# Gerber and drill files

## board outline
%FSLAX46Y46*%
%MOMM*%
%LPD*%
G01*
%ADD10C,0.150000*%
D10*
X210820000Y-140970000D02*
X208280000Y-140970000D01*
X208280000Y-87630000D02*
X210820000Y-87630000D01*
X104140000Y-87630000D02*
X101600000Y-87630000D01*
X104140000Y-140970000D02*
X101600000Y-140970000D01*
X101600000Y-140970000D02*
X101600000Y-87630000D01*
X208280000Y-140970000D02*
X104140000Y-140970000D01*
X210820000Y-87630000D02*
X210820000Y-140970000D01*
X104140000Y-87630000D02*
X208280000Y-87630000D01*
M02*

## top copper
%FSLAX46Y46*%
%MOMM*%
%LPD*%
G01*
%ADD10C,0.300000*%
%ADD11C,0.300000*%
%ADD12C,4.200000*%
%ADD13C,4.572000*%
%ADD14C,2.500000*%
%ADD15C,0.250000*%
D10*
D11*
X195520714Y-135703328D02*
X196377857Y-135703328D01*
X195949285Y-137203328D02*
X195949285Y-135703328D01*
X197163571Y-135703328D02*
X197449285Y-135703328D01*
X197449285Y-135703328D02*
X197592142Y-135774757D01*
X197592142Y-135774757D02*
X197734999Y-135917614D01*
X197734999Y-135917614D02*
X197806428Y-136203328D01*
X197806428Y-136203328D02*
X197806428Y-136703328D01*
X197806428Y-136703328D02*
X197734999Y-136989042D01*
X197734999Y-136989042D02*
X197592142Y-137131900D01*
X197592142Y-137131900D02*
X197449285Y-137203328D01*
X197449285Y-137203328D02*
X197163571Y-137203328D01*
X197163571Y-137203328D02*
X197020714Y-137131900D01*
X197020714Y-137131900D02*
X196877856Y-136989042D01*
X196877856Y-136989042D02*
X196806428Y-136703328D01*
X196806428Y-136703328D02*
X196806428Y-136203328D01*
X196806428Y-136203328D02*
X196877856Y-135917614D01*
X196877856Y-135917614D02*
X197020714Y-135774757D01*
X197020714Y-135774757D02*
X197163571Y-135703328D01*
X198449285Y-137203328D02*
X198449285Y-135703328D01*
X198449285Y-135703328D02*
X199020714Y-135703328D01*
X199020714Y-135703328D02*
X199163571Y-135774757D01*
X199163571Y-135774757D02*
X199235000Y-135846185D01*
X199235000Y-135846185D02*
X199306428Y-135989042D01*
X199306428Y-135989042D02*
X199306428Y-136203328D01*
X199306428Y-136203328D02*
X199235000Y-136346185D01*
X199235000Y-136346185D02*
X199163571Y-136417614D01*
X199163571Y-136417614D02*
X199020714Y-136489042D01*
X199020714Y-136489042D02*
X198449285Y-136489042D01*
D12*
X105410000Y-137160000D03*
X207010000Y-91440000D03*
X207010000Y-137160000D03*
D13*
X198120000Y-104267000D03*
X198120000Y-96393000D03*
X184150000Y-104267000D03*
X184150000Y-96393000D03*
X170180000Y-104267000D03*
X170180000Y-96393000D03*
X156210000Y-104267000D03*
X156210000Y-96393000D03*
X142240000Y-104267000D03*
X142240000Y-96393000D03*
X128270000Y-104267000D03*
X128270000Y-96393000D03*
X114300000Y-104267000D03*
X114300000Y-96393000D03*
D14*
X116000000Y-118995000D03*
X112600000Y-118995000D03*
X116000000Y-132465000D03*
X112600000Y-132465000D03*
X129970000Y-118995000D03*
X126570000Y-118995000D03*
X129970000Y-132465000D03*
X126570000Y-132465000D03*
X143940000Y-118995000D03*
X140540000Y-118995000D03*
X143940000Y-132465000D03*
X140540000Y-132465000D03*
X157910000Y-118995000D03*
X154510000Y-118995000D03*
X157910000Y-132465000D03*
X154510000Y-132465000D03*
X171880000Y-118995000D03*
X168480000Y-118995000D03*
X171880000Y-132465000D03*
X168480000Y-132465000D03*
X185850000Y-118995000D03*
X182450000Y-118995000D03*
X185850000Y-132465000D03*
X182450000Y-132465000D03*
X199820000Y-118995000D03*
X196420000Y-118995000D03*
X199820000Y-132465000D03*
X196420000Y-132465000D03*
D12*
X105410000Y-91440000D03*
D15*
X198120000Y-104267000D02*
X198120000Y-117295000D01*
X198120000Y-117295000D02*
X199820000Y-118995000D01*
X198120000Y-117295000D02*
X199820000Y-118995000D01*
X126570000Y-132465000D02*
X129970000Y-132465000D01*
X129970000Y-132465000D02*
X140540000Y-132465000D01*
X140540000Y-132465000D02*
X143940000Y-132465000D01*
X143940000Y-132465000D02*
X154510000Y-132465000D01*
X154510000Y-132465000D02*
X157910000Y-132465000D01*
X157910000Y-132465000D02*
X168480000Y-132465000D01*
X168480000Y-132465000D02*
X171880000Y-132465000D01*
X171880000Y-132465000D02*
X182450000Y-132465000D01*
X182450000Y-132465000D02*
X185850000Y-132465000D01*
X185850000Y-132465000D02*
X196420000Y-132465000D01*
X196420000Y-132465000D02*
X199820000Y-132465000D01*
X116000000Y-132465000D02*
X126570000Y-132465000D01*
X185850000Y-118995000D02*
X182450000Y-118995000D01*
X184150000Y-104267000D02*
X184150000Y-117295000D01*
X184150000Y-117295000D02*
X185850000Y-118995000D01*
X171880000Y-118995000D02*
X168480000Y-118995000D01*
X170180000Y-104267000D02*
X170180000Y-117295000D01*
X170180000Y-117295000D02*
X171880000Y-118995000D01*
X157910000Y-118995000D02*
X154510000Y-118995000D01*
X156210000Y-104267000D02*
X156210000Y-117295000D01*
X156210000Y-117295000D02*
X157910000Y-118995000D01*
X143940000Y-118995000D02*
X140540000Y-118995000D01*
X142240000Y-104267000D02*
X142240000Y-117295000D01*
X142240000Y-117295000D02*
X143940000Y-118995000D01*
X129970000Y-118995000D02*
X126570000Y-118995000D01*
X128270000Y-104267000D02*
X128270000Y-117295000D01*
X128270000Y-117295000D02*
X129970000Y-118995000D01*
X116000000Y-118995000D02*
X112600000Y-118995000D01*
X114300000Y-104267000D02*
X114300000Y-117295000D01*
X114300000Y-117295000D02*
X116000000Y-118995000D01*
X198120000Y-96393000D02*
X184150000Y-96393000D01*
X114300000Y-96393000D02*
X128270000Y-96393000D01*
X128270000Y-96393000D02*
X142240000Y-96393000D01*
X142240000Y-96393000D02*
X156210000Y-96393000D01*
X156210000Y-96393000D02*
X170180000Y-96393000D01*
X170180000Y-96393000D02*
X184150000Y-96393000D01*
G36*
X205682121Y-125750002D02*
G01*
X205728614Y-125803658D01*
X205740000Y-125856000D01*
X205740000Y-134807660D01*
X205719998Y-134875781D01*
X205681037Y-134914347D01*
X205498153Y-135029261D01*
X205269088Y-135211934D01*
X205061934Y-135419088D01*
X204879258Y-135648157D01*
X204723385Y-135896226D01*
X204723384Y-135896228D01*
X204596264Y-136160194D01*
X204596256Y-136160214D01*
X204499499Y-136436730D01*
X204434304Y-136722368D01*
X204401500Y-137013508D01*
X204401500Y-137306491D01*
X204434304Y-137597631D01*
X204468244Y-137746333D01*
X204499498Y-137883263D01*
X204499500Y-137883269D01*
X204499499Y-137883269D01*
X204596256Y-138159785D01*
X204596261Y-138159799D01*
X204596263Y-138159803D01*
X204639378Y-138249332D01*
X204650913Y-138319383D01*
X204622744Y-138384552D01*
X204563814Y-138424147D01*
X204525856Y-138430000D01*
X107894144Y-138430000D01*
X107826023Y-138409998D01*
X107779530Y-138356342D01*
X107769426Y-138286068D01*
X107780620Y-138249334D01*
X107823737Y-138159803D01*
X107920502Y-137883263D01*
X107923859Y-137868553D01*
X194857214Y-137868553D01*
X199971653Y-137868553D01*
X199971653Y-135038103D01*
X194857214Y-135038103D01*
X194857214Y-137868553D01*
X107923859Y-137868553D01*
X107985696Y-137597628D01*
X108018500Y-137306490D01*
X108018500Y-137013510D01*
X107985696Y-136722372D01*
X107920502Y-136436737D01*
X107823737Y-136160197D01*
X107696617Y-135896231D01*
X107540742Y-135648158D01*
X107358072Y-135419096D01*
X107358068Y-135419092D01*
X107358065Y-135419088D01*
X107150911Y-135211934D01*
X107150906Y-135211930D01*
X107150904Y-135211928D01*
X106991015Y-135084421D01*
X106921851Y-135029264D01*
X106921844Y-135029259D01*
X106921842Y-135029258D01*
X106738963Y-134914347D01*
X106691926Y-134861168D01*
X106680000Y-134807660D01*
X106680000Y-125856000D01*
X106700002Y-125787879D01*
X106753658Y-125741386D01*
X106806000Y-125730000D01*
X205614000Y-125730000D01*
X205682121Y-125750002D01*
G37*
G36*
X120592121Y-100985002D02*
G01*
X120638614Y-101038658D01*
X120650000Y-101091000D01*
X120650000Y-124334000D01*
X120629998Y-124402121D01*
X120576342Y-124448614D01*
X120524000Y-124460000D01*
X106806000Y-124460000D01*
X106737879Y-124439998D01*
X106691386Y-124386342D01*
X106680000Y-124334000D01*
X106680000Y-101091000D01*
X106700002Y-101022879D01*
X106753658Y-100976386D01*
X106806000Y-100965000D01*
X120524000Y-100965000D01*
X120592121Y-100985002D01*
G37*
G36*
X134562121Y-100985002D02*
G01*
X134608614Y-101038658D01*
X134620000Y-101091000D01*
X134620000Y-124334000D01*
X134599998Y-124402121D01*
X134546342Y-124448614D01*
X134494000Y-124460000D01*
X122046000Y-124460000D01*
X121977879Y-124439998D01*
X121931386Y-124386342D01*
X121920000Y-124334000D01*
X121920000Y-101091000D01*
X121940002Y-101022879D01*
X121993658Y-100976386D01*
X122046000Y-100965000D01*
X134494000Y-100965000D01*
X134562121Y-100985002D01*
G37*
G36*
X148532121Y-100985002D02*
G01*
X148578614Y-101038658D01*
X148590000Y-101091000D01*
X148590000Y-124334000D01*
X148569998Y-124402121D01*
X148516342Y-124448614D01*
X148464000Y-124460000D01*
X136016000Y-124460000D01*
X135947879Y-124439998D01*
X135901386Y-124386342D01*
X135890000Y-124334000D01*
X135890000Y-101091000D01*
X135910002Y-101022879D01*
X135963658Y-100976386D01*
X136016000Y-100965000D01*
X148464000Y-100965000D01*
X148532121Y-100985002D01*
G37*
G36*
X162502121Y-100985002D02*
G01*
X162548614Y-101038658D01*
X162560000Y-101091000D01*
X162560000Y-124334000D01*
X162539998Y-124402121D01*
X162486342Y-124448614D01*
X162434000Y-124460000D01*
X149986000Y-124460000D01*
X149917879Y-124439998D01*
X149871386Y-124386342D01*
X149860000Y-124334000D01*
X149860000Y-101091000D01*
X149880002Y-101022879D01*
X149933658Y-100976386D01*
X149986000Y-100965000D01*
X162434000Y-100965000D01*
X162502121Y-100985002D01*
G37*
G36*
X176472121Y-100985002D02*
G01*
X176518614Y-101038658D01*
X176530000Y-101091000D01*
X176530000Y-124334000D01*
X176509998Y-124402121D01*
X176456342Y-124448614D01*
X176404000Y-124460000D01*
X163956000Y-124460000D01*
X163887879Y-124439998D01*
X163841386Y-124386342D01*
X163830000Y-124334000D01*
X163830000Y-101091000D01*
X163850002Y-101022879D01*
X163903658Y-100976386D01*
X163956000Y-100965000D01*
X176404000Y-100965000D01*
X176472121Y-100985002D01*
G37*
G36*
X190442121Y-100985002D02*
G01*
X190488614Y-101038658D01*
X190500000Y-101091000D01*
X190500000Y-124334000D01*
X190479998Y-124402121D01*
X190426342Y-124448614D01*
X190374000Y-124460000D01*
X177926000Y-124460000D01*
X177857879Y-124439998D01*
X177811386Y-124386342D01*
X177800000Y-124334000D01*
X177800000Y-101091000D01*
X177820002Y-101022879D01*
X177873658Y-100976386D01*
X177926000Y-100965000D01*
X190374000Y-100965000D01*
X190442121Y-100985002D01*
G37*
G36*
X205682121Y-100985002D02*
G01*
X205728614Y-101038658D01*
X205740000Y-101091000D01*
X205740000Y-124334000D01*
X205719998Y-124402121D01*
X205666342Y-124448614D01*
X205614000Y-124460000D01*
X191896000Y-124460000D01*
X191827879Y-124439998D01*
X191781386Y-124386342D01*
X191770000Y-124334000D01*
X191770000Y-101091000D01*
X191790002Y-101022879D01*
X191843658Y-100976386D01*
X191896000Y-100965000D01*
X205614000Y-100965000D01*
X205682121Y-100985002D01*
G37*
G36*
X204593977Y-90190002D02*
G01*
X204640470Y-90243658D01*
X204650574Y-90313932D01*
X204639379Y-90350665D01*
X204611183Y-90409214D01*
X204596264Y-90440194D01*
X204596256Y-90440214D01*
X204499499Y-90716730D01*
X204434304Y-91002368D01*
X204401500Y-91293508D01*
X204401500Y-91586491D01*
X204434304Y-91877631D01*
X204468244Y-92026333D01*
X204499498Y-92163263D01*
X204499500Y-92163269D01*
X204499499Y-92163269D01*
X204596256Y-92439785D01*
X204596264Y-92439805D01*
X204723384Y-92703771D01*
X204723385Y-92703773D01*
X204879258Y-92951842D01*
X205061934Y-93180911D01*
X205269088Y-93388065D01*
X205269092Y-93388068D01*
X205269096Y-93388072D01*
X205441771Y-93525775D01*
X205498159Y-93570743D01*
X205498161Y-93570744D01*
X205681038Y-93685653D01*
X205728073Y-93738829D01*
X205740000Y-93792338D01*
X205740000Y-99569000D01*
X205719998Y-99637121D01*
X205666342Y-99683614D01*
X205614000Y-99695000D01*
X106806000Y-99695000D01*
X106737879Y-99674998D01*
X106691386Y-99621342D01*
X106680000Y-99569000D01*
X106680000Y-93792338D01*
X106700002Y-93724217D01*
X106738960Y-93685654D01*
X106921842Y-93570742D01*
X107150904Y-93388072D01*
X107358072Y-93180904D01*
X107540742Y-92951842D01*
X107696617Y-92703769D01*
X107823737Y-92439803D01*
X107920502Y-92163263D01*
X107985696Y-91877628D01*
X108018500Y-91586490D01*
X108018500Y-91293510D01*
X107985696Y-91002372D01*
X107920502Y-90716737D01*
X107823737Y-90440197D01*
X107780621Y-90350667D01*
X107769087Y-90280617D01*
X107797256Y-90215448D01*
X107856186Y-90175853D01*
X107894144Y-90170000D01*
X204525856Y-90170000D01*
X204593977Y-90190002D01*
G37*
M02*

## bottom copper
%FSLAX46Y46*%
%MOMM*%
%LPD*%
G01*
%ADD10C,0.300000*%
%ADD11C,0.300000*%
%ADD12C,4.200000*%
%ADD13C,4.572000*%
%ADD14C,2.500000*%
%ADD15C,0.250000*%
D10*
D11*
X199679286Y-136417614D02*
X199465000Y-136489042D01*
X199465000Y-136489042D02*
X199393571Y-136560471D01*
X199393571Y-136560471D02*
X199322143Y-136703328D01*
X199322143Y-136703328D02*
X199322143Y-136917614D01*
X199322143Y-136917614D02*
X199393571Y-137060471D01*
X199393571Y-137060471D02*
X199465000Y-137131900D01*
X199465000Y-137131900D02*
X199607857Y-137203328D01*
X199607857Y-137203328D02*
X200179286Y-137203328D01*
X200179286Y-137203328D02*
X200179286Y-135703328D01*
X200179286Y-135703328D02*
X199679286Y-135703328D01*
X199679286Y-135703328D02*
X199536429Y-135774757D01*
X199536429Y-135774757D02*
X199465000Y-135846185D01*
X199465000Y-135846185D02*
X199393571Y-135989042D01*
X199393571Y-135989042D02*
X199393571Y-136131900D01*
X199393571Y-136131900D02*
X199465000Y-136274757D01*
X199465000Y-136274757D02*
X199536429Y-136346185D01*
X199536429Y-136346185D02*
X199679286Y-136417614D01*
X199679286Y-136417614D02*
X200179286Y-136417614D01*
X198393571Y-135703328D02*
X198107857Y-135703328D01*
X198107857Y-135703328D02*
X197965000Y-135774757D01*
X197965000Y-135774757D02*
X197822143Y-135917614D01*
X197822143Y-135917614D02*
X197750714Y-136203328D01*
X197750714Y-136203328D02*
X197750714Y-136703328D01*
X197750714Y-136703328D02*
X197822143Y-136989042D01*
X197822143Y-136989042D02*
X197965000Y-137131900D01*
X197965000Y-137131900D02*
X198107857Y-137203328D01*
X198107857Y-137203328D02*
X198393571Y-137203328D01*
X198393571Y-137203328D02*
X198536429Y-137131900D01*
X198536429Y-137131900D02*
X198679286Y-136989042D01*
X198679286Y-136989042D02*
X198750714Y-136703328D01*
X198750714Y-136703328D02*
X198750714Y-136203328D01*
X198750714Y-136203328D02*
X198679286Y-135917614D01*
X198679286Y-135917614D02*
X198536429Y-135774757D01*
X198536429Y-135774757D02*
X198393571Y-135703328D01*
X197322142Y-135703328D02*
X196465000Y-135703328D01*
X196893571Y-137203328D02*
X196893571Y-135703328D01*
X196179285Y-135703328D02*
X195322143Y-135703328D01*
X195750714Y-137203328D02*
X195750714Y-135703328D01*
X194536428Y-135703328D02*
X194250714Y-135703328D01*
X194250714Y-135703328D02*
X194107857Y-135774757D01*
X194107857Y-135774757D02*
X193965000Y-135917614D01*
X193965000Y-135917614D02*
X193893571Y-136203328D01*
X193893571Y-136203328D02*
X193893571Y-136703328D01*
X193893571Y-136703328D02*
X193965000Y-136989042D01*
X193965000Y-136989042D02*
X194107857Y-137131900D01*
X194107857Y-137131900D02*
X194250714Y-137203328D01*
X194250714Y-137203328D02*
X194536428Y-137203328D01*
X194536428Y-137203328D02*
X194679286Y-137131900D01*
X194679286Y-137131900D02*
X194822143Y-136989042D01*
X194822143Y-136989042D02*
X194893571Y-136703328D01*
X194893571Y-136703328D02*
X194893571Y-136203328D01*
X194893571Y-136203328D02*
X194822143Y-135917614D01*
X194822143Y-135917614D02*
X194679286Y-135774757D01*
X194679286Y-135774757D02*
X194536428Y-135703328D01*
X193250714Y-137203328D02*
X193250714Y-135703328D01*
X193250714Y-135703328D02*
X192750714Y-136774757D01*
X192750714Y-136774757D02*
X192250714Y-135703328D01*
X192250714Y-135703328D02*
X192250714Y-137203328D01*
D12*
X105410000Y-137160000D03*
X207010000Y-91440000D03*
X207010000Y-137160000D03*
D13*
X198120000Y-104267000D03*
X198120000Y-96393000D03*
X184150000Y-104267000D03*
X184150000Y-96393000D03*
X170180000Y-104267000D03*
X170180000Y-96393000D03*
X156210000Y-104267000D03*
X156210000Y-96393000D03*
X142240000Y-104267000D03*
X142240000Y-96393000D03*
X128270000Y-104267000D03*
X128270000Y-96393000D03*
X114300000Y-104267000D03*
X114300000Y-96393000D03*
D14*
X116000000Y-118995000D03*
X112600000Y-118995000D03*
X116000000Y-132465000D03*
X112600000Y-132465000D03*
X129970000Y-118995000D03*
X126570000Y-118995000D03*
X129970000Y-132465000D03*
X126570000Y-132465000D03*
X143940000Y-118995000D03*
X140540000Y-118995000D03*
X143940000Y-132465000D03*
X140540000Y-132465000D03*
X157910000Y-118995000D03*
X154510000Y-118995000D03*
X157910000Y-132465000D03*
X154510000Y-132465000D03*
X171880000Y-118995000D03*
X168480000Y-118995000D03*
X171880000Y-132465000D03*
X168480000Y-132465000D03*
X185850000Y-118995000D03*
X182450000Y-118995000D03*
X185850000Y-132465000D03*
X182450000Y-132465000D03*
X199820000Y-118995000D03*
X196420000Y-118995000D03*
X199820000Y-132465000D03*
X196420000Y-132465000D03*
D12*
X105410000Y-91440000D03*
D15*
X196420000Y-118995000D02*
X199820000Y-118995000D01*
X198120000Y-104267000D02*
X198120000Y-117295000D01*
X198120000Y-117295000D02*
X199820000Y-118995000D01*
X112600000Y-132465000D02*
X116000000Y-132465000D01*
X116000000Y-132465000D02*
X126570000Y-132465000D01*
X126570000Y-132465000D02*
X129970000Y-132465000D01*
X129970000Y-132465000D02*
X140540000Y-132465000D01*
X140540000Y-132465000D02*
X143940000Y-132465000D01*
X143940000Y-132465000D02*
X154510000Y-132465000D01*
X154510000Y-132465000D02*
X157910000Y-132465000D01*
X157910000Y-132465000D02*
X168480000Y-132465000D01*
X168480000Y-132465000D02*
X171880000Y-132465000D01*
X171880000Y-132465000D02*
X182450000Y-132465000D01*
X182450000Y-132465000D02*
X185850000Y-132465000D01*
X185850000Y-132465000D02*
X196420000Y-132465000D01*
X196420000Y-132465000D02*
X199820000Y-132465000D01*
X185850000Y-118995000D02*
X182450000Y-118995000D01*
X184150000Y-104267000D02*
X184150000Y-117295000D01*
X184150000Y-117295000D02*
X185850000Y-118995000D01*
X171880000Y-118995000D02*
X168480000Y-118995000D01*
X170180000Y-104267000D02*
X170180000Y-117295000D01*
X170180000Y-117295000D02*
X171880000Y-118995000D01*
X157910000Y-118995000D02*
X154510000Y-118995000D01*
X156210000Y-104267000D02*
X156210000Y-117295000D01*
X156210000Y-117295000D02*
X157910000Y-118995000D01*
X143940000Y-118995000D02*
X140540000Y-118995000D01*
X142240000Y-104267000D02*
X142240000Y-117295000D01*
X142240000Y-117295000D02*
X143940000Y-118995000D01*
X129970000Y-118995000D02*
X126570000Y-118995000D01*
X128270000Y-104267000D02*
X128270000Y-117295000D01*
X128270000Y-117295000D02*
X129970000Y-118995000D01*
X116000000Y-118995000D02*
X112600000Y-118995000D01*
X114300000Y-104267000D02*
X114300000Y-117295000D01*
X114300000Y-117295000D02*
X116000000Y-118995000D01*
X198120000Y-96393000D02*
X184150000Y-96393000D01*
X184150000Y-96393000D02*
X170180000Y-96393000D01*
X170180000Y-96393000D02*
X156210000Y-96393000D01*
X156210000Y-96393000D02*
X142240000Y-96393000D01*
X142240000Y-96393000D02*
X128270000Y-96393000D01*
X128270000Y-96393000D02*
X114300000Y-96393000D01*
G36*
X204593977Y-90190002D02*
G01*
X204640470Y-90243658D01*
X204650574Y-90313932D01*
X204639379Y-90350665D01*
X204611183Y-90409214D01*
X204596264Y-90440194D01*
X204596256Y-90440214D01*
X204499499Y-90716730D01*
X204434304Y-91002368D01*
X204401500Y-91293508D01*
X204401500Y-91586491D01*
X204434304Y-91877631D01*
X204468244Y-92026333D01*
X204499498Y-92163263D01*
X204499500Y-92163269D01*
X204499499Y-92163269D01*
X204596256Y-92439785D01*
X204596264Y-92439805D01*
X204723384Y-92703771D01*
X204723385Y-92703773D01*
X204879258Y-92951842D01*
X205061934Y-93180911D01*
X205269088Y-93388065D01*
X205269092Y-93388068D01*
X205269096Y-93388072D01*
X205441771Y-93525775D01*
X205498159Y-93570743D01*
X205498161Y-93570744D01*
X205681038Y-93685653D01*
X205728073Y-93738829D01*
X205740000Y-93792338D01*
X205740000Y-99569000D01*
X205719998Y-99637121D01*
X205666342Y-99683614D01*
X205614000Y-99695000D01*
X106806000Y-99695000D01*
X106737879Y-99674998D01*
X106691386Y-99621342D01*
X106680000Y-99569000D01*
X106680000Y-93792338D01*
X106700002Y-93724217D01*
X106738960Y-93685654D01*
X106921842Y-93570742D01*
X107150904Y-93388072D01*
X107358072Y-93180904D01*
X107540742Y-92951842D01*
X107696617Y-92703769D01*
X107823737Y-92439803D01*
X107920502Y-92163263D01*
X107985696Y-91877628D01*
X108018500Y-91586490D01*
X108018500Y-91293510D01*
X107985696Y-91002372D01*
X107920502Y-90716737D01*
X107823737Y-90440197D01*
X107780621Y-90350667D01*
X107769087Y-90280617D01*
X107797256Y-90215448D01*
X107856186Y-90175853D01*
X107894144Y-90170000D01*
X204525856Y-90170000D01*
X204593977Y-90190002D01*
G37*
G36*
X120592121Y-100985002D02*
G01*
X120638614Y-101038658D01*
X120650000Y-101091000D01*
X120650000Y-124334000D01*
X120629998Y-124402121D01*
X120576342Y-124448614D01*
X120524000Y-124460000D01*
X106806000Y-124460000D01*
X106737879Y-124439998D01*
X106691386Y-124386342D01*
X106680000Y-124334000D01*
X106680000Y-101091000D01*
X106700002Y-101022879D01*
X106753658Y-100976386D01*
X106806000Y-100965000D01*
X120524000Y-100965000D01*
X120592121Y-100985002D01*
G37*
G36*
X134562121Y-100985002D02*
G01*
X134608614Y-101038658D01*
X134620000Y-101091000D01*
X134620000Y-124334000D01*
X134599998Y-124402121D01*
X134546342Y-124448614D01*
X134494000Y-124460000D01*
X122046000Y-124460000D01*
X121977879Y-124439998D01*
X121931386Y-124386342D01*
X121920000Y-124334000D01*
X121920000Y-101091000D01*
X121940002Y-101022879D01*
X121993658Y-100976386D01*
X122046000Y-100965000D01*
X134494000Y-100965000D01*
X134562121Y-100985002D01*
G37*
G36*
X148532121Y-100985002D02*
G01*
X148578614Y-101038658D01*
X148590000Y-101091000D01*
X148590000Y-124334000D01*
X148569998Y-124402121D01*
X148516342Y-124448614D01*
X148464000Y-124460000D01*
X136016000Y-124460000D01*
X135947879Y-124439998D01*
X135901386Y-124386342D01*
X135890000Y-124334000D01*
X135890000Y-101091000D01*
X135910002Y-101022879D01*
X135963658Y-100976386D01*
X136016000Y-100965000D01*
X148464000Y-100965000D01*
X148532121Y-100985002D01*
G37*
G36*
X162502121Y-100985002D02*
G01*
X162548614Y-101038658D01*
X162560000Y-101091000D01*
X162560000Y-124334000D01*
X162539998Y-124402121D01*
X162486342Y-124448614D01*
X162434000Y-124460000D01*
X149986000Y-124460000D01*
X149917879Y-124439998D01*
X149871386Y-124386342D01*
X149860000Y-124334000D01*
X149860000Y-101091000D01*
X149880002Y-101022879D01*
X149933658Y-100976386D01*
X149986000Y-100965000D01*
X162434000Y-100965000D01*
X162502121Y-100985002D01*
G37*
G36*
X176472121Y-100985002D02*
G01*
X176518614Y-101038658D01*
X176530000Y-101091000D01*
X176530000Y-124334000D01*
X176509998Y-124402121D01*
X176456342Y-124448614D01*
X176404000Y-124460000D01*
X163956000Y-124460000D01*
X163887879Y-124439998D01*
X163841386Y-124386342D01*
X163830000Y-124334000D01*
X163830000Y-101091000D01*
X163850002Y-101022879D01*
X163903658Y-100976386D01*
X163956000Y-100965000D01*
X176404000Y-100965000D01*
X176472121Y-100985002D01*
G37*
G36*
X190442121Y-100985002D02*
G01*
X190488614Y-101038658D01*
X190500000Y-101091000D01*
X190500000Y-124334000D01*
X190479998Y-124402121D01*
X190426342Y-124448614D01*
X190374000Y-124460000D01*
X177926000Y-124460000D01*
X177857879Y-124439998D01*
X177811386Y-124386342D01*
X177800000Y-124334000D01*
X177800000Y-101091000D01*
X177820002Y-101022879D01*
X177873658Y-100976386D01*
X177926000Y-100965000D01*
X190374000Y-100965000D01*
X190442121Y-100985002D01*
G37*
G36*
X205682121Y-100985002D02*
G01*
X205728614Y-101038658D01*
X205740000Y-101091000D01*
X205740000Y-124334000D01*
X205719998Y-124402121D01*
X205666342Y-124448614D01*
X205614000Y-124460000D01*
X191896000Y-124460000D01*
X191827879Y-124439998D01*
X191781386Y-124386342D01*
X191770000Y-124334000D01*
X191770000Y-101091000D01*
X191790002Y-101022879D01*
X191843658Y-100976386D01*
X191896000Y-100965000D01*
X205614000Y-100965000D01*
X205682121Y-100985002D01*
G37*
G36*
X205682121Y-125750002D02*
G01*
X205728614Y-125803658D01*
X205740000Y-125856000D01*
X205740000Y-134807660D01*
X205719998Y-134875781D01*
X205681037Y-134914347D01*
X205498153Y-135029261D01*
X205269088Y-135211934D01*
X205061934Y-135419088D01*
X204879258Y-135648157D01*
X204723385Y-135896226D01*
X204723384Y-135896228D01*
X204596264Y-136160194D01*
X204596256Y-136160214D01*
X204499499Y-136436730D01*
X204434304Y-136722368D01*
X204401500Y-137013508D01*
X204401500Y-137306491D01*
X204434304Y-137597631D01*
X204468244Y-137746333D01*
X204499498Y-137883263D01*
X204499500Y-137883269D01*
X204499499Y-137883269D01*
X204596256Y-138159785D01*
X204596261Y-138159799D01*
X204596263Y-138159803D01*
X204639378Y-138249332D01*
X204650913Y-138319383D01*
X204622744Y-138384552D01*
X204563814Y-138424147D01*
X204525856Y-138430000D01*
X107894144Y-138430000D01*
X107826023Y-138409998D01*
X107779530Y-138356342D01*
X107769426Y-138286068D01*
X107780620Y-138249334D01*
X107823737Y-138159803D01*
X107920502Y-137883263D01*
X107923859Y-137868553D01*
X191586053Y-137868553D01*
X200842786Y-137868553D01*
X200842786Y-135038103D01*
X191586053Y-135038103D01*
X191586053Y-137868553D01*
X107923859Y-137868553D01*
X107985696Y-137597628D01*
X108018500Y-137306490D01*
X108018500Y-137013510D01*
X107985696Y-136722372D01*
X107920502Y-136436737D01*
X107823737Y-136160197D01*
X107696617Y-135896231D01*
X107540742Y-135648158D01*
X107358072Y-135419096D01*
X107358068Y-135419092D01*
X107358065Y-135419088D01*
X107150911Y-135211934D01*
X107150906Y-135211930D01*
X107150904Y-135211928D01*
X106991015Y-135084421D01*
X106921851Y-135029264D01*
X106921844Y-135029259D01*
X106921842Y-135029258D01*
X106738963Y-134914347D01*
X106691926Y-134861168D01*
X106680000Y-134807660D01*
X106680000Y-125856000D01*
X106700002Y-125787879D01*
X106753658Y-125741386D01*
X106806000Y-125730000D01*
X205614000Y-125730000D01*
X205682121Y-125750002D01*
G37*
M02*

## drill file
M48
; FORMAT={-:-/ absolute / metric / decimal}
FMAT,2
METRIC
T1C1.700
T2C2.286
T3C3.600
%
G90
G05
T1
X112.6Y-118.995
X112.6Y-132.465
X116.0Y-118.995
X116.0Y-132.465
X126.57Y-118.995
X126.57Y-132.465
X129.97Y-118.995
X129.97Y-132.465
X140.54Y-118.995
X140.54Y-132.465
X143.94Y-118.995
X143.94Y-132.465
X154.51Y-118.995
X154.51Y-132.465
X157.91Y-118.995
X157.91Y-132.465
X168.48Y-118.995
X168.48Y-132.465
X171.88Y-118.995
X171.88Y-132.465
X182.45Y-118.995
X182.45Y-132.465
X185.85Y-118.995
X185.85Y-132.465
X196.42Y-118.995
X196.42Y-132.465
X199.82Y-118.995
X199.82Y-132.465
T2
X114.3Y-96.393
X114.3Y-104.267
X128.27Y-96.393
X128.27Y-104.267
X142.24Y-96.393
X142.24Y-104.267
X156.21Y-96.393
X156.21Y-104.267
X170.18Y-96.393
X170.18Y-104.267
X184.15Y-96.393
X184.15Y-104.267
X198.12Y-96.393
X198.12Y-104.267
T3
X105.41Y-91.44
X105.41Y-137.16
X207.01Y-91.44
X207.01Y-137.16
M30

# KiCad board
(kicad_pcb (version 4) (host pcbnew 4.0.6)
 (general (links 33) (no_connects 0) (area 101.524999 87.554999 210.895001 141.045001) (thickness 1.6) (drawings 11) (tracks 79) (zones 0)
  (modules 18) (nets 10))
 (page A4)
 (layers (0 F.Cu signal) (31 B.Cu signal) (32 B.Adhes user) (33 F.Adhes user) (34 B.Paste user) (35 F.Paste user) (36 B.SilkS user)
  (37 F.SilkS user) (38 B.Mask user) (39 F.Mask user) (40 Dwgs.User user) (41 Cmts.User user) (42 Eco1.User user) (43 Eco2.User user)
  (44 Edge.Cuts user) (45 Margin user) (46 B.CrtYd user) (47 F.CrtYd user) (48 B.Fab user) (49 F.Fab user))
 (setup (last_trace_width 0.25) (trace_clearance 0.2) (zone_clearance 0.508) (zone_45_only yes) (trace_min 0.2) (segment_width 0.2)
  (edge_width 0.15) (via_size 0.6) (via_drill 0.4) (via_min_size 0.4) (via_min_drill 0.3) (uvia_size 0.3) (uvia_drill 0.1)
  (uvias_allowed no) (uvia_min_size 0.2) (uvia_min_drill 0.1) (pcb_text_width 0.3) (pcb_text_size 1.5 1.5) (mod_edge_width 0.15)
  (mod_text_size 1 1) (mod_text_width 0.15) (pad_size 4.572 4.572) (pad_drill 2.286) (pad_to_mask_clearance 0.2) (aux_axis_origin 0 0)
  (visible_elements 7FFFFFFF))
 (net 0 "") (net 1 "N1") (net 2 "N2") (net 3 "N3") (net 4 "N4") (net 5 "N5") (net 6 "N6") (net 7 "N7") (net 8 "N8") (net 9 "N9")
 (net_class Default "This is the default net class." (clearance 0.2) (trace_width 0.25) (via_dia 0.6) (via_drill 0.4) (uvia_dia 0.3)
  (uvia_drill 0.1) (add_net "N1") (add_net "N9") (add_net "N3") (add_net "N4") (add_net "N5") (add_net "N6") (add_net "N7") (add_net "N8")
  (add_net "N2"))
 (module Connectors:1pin (layer F.Cu) (at 105.41 137.16)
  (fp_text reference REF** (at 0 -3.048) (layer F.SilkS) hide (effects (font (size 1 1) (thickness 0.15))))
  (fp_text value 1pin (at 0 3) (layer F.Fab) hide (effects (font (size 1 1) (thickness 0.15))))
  (pad 1 thru_hole circle (at 0 0) (size 4.2 4.2) (drill 3.6) (layers *.Cu *.Mask)))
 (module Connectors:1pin (layer F.Cu) (at 207.01 91.44)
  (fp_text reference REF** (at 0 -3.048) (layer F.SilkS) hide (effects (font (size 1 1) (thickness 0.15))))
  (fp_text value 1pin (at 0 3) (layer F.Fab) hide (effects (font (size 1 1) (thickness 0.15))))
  (pad 1 thru_hole circle (at 0 0) (size 4.2 4.2) (drill 3.6) (layers *.Cu *.Mask)))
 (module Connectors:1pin (layer F.Cu) (at 207.01 137.16)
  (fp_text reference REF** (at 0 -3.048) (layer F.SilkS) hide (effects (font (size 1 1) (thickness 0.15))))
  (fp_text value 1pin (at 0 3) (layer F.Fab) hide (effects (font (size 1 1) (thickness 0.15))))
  (pad 1 thru_hole circle (at 0 0) (size 4.2 4.2) (drill 3.6) (layers *.Cu *.Mask)))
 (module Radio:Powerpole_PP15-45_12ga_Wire (layer F.Cu) (at 198.12 100.33 90)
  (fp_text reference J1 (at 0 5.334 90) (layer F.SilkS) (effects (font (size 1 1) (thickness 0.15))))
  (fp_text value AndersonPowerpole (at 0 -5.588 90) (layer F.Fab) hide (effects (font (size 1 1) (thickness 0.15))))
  (pad 1 thru_hole circle (at -3.937 0 90) (size 4.572 4.572) (drill 2.286) (layers *.Cu *.Mask) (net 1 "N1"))
  (pad 2 thru_hole circle (at 3.937 0 90) (size 4.572 4.572) (drill 2.286) (layers *.Cu *.Mask) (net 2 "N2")))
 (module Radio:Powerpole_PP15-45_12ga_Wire (layer F.Cu) (at 184.15 100.33 90)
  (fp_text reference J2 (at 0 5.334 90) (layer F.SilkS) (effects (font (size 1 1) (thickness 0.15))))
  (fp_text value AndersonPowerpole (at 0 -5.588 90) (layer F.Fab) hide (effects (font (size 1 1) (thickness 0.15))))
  (pad 1 thru_hole circle (at -3.937 0 90) (size 4.572 4.572) (drill 2.286) (layers *.Cu *.Mask) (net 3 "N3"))
  (pad 2 thru_hole circle (at 3.937 0 90) (size 4.572 4.572) (drill 2.286) (layers *.Cu *.Mask) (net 2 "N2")))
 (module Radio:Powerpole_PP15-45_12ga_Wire (layer F.Cu) (at 170.18 100.33 90)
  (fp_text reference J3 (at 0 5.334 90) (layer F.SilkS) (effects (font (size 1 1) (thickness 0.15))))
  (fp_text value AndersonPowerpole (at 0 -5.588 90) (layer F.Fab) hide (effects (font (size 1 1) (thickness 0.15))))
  (pad 1 thru_hole circle (at -3.937 0 90) (size 4.572 4.572) (drill 2.286) (layers *.Cu *.Mask) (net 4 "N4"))
  (pad 2 thru_hole circle (at 3.937 0 90) (size 4.572 4.572) (drill 2.286) (layers *.Cu *.Mask) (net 2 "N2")))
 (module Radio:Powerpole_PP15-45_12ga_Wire (layer F.Cu) (at 156.21 100.33 90)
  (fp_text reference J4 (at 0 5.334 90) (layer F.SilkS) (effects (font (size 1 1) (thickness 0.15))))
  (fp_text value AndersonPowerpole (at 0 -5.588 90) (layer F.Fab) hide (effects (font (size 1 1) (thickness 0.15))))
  (pad 1 thru_hole circle (at -3.937 0 90) (size 4.572 4.572) (drill 2.286) (layers *.Cu *.Mask) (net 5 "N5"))
  (pad 2 thru_hole circle (at 3.937 0 90) (size 4.572 4.572) (drill 2.286) (layers *.Cu *.Mask) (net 2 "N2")))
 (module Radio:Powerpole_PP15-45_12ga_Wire (layer F.Cu) (at 142.24 100.33 90)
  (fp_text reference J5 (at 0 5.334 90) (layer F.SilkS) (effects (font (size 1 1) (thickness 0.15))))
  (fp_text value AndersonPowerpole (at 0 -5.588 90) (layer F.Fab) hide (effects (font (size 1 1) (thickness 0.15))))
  (pad 1 thru_hole circle (at -3.937 0 90) (size 4.572 4.572) (drill 2.286) (layers *.Cu *.Mask) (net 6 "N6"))
  (pad 2 thru_hole circle (at 3.937 0 90) (size 4.572 4.572) (drill 2.286) (layers *.Cu *.Mask) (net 2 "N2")))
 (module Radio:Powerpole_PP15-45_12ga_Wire (layer F.Cu) (at 128.27 100.33 90)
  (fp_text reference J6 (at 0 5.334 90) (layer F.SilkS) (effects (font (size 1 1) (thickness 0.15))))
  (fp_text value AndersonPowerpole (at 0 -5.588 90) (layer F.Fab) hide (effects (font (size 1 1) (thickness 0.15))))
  (pad 1 thru_hole circle (at -3.937 0 90) (size 4.572 4.572) (drill 2.286) (layers *.Cu *.Mask) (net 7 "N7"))
  (pad 2 thru_hole circle (at 3.937 0 90) (size 4.572 4.572) (drill 2.286) (layers *.Cu *.Mask) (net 2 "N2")))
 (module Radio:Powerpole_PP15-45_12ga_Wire (layer F.Cu) (at 114.3 100.33 90)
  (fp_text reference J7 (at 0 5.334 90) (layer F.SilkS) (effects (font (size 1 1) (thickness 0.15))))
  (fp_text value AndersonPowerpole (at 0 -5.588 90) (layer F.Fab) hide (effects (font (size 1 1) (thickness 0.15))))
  (pad 1 thru_hole circle (at -3.937 0 90) (size 4.572 4.572) (drill 2.286) (layers *.Cu *.Mask) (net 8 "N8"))
  (pad 2 thru_hole circle (at 3.937 0 90) (size 4.572 4.572) (drill 2.286) (layers *.Cu *.Mask) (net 2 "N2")))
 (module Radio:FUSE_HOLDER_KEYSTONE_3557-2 (layer F.Cu) (at 114.3 125.73 270)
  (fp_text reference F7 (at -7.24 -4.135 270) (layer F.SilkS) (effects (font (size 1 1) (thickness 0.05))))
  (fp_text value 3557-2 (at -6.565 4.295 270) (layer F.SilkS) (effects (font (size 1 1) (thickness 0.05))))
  (pad 1 thru_hole circle (at -6.735 -1.7 270) (size 2.5 2.5) (drill 1.7) (layers *.Cu *.Mask F.SilkS) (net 8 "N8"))
  (pad 2 thru_hole circle (at -6.735 1.7 270) (size 2.5 2.5) (drill 1.7) (layers *.Cu *.Mask F.SilkS) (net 8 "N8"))
  (pad 3 thru_hole circle (at 6.735 -1.7 270) (size 2.5 2.5) (drill 1.7) (layers *.Cu *.Mask F.SilkS) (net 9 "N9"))
  (pad 4 thru_hole circle (at 6.735 1.7 270) (size 2.5 2.5) (drill 1.7) (layers *.Cu *.Mask F.SilkS) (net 9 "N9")))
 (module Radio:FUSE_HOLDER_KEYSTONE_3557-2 (layer F.Cu) (at 128.27 125.73 270)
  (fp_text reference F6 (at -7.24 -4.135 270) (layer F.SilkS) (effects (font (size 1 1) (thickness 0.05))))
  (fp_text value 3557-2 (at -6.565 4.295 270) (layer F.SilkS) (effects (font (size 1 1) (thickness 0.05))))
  (pad 1 thru_hole circle (at -6.735 -1.7 270) (size 2.5 2.5) (drill 1.7) (layers *.Cu *.Mask F.SilkS) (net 7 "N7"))
  (pad 2 thru_hole circle (at -6.735 1.7 270) (size 2.5 2.5) (drill 1.7) (layers *.Cu *.Mask F.SilkS) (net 7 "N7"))
  (pad 3 thru_hole circle (at 6.735 -1.7 270) (size 2.5 2.5) (drill 1.7) (layers *.Cu *.Mask F.SilkS) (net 9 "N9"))
  (pad 4 thru_hole circle (at 6.735 1.7 270) (size 2.5 2.5) (drill 1.7) (layers *.Cu *.Mask F.SilkS) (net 9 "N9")))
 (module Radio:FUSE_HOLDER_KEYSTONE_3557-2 (layer F.Cu) (at 142.24 125.73 270)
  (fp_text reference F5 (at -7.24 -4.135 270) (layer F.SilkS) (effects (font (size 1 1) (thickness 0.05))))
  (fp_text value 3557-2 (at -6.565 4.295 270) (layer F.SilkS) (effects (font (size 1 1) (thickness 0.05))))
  (pad 1 thru_hole circle (at -6.735 -1.7 270) (size 2.5 2.5) (drill 1.7) (layers *.Cu *.Mask F.SilkS) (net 6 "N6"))
  (pad 2 thru_hole circle (at -6.735 1.7 270) (size 2.5 2.5) (drill 1.7) (layers *.Cu *.Mask F.SilkS) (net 6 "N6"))
  (pad 3 thru_hole circle (at 6.735 -1.7 270) (size 2.5 2.5) (drill 1.7) (layers *.Cu *.Mask F.SilkS) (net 9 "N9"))
  (pad 4 thru_hole circle (at 6.735 1.7 270) (size 2.5 2.5) (drill 1.7) (layers *.Cu *.Mask F.SilkS) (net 9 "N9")))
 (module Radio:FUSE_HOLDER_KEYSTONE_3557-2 (layer F.Cu) (at 156.21 125.73 270)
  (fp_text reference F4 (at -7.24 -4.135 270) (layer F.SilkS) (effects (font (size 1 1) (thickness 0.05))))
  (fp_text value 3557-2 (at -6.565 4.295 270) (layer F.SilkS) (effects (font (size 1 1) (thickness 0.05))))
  (pad 1 thru_hole circle (at -6.735 -1.7 270) (size 2.5 2.5) (drill 1.7) (layers *.Cu *.Mask F.SilkS) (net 5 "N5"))
  (pad 2 thru_hole circle (at -6.735 1.7 270) (size 2.5 2.5) (drill 1.7) (layers *.Cu *.Mask F.SilkS) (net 5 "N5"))
  (pad 3 thru_hole circle (at 6.735 -1.7 270) (size 2.5 2.5) (drill 1.7) (layers *.Cu *.Mask F.SilkS) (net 9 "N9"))
  (pad 4 thru_hole circle (at 6.735 1.7 270) (size 2.5 2.5) (drill 1.7) (layers *.Cu *.Mask F.SilkS) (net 9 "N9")))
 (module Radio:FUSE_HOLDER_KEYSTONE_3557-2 (layer F.Cu) (at 170.18 125.73 270)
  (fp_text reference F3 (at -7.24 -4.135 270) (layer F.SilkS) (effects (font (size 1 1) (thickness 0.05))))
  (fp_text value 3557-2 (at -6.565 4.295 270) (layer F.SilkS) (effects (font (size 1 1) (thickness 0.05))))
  (pad 1 thru_hole circle (at -6.735 -1.7 270) (size 2.5 2.5) (drill 1.7) (layers *.Cu *.Mask F.SilkS) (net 4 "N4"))
  (pad 2 thru_hole circle (at -6.735 1.7 270) (size 2.5 2.5) (drill 1.7) (layers *.Cu *.Mask F.SilkS) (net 4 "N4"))
  (pad 3 thru_hole circle (at 6.735 -1.7 270) (size 2.5 2.5) (drill 1.7) (layers *.Cu *.Mask F.SilkS) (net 9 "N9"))
  (pad 4 thru_hole circle (at 6.735 1.7 270) (size 2.5 2.5) (drill 1.7) (layers *.Cu *.Mask F.SilkS) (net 9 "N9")))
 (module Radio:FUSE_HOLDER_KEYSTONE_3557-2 (layer F.Cu) (at 184.15 125.73 270)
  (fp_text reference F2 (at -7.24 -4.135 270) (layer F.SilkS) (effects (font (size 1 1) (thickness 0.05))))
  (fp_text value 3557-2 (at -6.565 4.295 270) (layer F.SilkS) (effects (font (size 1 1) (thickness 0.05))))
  (pad 1 thru_hole circle (at -6.735 -1.7 270) (size 2.5 2.5) (drill 1.7) (layers *.Cu *.Mask F.SilkS) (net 3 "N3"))
  (pad 2 thru_hole circle (at -6.735 1.7 270) (size 2.5 2.5) (drill 1.7) (layers *.Cu *.Mask F.SilkS) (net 3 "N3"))
  (pad 3 thru_hole circle (at 6.735 -1.7 270) (size 2.5 2.5) (drill 1.7) (layers *.Cu *.Mask F.SilkS) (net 9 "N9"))
  (pad 4 thru_hole circle (at 6.735 1.7 270) (size 2.5 2.5) (drill 1.7) (layers *.Cu *.Mask F.SilkS) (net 9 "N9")))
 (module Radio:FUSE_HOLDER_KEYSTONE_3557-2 (layer F.Cu) (at 198.12 125.73 270)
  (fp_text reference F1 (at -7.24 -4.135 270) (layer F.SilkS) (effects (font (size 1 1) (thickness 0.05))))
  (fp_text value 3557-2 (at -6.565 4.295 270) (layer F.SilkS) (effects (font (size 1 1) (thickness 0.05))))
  (pad 1 thru_hole circle (at -6.735 -1.7 270) (size 2.5 2.5) (drill 1.7) (layers *.Cu *.Mask F.SilkS) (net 1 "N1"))
  (pad 2 thru_hole circle (at -6.735 1.7 270) (size 2.5 2.5) (drill 1.7) (layers *.Cu *.Mask F.SilkS) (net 1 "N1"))
  (pad 3 thru_hole circle (at 6.735 -1.7 270) (size 2.5 2.5) (drill 1.7) (layers *.Cu *.Mask F.SilkS) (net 9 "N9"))
  (pad 4 thru_hole circle (at 6.735 1.7 270) (size 2.5 2.5) (drill 1.7) (layers *.Cu *.Mask F.SilkS) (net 9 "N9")))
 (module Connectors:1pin (layer F.Cu) (at 105.41 91.44)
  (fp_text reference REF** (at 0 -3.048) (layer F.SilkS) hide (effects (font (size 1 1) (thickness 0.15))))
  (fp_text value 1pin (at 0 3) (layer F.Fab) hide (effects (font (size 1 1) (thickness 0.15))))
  (pad 1 thru_hole circle (at 0 0) (size 4.2 4.2) (drill 3.6) (layers *.Cu *.Mask)))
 (gr_line (start 210.82 140.97) (end 208.28 140.97) (angle 90) (layer Edge.Cuts) (width 0.15))
 (gr_line (start 208.28 87.63) (end 210.82 87.63) (angle 90) (layer Edge.Cuts) (width 0.15))
 (gr_line (start 104.14 87.63) (end 101.6 87.63) (angle 90) (layer Edge.Cuts) (width 0.15))
 (gr_line (start 104.14 140.97) (end 101.6 140.97) (angle 90) (layer Edge.Cuts) (width 0.15))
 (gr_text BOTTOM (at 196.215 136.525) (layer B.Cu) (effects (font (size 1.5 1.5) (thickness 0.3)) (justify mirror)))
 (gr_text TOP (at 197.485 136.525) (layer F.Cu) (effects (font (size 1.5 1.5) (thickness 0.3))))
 (gr_line (start 101.6 140.97) (end 101.6 87.63) (angle 90) (layer Edge.Cuts) (width 0.15))
 (gr_line (start 208.28 140.97) (end 104.14 140.97) (angle 90) (layer Edge.Cuts) (width 0.15))
 (gr_line (start 210.82 87.63) (end 210.82 140.97) (angle 90) (layer Edge.Cuts) (width 0.15))
 (gr_line (start 104.14 87.63) (end 208.28 87.63) (angle 90) (layer Edge.Cuts) (width 0.15))
 (segment (start 196.42 118.995) (end 199.82 118.995) (width 0.25) (layer B.Cu) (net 1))
 (segment (start 198.12 104.267) (end 198.12 117.295) (width 0.25) (layer F.Cu) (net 1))
 (segment (start 198.12 104.267) (end 198.12 117.295) (width 0.25) (layer B.Cu) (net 1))
 (segment (start 198.12 117.295) (end 199.82 118.995) (width 0.25) (layer B.Cu) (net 1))
 (segment (start 198.12 117.295) (end 199.82 118.995) (width 0.25) (layer F.Cu) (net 1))
 (segment (start 198.12 117.295) (end 199.82 118.995) (width 0.25) (layer F.Cu) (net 1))
 (segment (start 112.6 132.465) (end 116 132.465) (width 0.25) (layer B.Cu) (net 9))
 (segment (start 116 132.465) (end 126.57 132.465) (width 0.25) (layer B.Cu) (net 9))
 (segment (start 126.57 132.465) (end 129.97 132.465) (width 0.25) (layer B.Cu) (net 9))
 (segment (start 129.97 132.465) (end 140.54 132.465) (width 0.25) (layer B.Cu) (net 9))
 (segment (start 140.54 132.465) (end 143.94 132.465) (width 0.25) (layer B.Cu) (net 9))
 (segment (start 143.94 132.465) (end 154.51 132.465) (width 0.25) (layer B.Cu) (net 9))
 (segment (start 154.51 132.465) (end 157.91 132.465) (width 0.25) (layer B.Cu) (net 9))
 (segment (start 157.91 132.465) (end 168.48 132.465) (width 0.25) (layer B.Cu) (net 9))
 (segment (start 168.48 132.465) (end 171.88 132.465) (width 0.25) (layer B.Cu) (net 9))
 (segment (start 171.88 132.465) (end 182.45 132.465) (width 0.25) (layer B.Cu) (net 9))
 (segment (start 182.45 132.465) (end 185.85 132.465) (width 0.25) (layer B.Cu) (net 9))
 (segment (start 185.85 132.465) (end 196.42 132.465) (width 0.25) (layer B.Cu) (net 9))
 (segment (start 196.42 132.465) (end 199.82 132.465) (width 0.25) (layer B.Cu) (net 9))
 (segment (start 126.57 132.465) (end 129.97 132.465) (width 0.25) (layer F.Cu) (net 9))
 (segment (start 129.97 132.465) (end 140.54 132.465) (width 0.25) (layer F.Cu) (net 9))
 (segment (start 140.54 132.465) (end 143.94 132.465) (width 0.25) (layer F.Cu) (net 9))
 (segment (start 143.94 132.465) (end 154.51 132.465) (width 0.25) (layer F.Cu) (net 9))
 (segment (start 154.51 132.465) (end 157.91 132.465) (width 0.25) (layer F.Cu) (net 9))
 (segment (start 157.91 132.465) (end 168.48 132.465) (width 0.25) (layer F.Cu) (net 9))
 (segment (start 168.48 132.465) (end 171.88 132.465) (width 0.25) (layer F.Cu) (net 9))
 (segment (start 171.88 132.465) (end 182.45 132.465) (width 0.25) (layer F.Cu) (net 9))
 (segment (start 182.45 132.465) (end 185.85 132.465) (width 0.25) (layer F.Cu) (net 9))
 (segment (start 185.85 132.465) (end 196.42 132.465) (width 0.25) (layer F.Cu) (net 9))
 (segment (start 196.42 132.465) (end 199.82 132.465) (width 0.25) (layer F.Cu) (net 9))
 (segment (start 116 132.465) (end 126.57 132.465) (width 0.25) (layer F.Cu) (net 9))
 (segment (start 185.85 118.995) (end 182.45 118.995) (width 0.25) (layer B.Cu) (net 3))
 (segment (start 184.15 104.267) (end 184.15 117.295) (width 0.25) (layer B.Cu) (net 3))
 (segment (start 184.15 117.295) (end 185.85 118.995) (width 0.25) (layer B.Cu) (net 3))
 (segment (start 185.85 118.995) (end 182.45 118.995) (width 0.25) (layer F.Cu) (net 3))
 (segment (start 184.15 104.267) (end 184.15 117.295) (width 0.25) (layer F.Cu) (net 3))
 (segment (start 184.15 117.295) (end 185.85 118.995) (width 0.25) (layer F.Cu) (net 3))
 (segment (start 171.88 118.995) (end 168.48 118.995) (width 0.25) (layer B.Cu) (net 4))
 (segment (start 170.18 104.267) (end 170.18 117.295) (width 0.25) (layer B.Cu) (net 4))
 (segment (start 170.18 117.295) (end 171.88 118.995) (width 0.25) (layer B.Cu) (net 4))
 (segment (start 171.88 118.995) (end 168.48 118.995) (width 0.25) (layer F.Cu) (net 4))
 (segment (start 170.18 104.267) (end 170.18 117.295) (width 0.25) (layer F.Cu) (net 4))
 (segment (start 170.18 117.295) (end 171.88 118.995) (width 0.25) (layer F.Cu) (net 4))
 (segment (start 157.91 118.995) (end 154.51 118.995) (width 0.25) (layer B.Cu) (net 5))
 (segment (start 156.21 104.267) (end 156.21 117.295) (width 0.25) (layer B.Cu) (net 5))
 (segment (start 156.21 117.295) (end 157.91 118.995) (width 0.25) (layer B.Cu) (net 5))
 (segment (start 157.91 118.995) (end 154.51 118.995) (width 0.25) (layer F.Cu) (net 5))
 (segment (start 156.21 104.267) (end 156.21 117.295) (width 0.25) (layer F.Cu) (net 5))
 (segment (start 156.21 117.295) (end 157.91 118.995) (width 0.25) (layer F.Cu) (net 5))
 (segment (start 143.94 118.995) (end 140.54 118.995) (width 0.25) (layer B.Cu) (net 6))
 (segment (start 142.24 104.267) (end 142.24 117.295) (width 0.25) (layer B.Cu) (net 6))
 (segment (start 142.24 117.295) (end 143.94 118.995) (width 0.25) (layer B.Cu) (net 6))
 (segment (start 143.94 118.995) (end 140.54 118.995) (width 0.25) (layer F.Cu) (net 6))
 (segment (start 142.24 104.267) (end 142.24 117.295) (width 0.25) (layer F.Cu) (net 6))
 (segment (start 142.24 117.295) (end 143.94 118.995) (width 0.25) (layer F.Cu) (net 6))
 (segment (start 129.97 118.995) (end 126.57 118.995) (width 0.25) (layer B.Cu) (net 7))
 (segment (start 128.27 104.267) (end 128.27 117.295) (width 0.25) (layer B.Cu) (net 7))
 (segment (start 128.27 117.295) (end 129.97 118.995) (width 0.25) (layer B.Cu) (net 7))
 (segment (start 129.97 118.995) (end 126.57 118.995) (width 0.25) (layer F.Cu) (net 7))
 (segment (start 128.27 104.267) (end 128.27 117.295) (width 0.25) (layer F.Cu) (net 7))
 (segment (start 128.27 117.295) (end 129.97 118.995) (width 0.25) (layer F.Cu) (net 7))
 (segment (start 116 118.995) (end 112.6 118.995) (width 0.25) (layer B.Cu) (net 8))
 (segment (start 114.3 104.267) (end 114.3 117.295) (width 0.25) (layer B.Cu) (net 8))
 (segment (start 114.3 117.295) (end 116 118.995) (width 0.25) (layer B.Cu) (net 8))
 (segment (start 116 118.995) (end 112.6 118.995) (width 0.25) (layer F.Cu) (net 8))
 (segment (start 114.3 104.267) (end 114.3 117.295) (width 0.25) (layer F.Cu) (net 8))
 (segment (start 114.3 117.295) (end 116 118.995) (width 0.25) (layer F.Cu) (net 8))
 (segment (start 198.12 96.393) (end 184.15 96.393) (width 0.25) (layer B.Cu) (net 2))
 (segment (start 198.12 96.393) (end 184.15 96.393) (width 0.25) (layer F.Cu) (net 2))
 (segment (start 184.15 96.393) (end 170.18 96.393) (width 0.25) (layer B.Cu) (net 2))
 (segment (start 170.18 96.393) (end 156.21 96.393) (width 0.25) (layer B.Cu) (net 2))
 (segment (start 156.21 96.393) (end 142.24 96.393) (width 0.25) (layer B.Cu) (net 2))
 (segment (start 142.24 96.393) (end 128.27 96.393) (width 0.25) (layer B.Cu) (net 2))
 (segment (start 128.27 96.393) (end 114.3 96.393) (width 0.25) (layer B.Cu) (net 2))
 (segment (start 114.3 96.393) (end 128.27 96.393) (width 0.25) (layer F.Cu) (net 2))
 (segment (start 128.27 96.393) (end 142.24 96.393) (width 0.25) (layer F.Cu) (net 2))
 (segment (start 142.24 96.393) (end 156.21 96.393) (width 0.25) (layer F.Cu) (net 2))
 (segment (start 156.21 96.393) (end 170.18 96.393) (width 0.25) (layer F.Cu) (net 2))
 (segment (start 170.18 96.393) (end 184.15 96.393) (width 0.25) (layer F.Cu) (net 2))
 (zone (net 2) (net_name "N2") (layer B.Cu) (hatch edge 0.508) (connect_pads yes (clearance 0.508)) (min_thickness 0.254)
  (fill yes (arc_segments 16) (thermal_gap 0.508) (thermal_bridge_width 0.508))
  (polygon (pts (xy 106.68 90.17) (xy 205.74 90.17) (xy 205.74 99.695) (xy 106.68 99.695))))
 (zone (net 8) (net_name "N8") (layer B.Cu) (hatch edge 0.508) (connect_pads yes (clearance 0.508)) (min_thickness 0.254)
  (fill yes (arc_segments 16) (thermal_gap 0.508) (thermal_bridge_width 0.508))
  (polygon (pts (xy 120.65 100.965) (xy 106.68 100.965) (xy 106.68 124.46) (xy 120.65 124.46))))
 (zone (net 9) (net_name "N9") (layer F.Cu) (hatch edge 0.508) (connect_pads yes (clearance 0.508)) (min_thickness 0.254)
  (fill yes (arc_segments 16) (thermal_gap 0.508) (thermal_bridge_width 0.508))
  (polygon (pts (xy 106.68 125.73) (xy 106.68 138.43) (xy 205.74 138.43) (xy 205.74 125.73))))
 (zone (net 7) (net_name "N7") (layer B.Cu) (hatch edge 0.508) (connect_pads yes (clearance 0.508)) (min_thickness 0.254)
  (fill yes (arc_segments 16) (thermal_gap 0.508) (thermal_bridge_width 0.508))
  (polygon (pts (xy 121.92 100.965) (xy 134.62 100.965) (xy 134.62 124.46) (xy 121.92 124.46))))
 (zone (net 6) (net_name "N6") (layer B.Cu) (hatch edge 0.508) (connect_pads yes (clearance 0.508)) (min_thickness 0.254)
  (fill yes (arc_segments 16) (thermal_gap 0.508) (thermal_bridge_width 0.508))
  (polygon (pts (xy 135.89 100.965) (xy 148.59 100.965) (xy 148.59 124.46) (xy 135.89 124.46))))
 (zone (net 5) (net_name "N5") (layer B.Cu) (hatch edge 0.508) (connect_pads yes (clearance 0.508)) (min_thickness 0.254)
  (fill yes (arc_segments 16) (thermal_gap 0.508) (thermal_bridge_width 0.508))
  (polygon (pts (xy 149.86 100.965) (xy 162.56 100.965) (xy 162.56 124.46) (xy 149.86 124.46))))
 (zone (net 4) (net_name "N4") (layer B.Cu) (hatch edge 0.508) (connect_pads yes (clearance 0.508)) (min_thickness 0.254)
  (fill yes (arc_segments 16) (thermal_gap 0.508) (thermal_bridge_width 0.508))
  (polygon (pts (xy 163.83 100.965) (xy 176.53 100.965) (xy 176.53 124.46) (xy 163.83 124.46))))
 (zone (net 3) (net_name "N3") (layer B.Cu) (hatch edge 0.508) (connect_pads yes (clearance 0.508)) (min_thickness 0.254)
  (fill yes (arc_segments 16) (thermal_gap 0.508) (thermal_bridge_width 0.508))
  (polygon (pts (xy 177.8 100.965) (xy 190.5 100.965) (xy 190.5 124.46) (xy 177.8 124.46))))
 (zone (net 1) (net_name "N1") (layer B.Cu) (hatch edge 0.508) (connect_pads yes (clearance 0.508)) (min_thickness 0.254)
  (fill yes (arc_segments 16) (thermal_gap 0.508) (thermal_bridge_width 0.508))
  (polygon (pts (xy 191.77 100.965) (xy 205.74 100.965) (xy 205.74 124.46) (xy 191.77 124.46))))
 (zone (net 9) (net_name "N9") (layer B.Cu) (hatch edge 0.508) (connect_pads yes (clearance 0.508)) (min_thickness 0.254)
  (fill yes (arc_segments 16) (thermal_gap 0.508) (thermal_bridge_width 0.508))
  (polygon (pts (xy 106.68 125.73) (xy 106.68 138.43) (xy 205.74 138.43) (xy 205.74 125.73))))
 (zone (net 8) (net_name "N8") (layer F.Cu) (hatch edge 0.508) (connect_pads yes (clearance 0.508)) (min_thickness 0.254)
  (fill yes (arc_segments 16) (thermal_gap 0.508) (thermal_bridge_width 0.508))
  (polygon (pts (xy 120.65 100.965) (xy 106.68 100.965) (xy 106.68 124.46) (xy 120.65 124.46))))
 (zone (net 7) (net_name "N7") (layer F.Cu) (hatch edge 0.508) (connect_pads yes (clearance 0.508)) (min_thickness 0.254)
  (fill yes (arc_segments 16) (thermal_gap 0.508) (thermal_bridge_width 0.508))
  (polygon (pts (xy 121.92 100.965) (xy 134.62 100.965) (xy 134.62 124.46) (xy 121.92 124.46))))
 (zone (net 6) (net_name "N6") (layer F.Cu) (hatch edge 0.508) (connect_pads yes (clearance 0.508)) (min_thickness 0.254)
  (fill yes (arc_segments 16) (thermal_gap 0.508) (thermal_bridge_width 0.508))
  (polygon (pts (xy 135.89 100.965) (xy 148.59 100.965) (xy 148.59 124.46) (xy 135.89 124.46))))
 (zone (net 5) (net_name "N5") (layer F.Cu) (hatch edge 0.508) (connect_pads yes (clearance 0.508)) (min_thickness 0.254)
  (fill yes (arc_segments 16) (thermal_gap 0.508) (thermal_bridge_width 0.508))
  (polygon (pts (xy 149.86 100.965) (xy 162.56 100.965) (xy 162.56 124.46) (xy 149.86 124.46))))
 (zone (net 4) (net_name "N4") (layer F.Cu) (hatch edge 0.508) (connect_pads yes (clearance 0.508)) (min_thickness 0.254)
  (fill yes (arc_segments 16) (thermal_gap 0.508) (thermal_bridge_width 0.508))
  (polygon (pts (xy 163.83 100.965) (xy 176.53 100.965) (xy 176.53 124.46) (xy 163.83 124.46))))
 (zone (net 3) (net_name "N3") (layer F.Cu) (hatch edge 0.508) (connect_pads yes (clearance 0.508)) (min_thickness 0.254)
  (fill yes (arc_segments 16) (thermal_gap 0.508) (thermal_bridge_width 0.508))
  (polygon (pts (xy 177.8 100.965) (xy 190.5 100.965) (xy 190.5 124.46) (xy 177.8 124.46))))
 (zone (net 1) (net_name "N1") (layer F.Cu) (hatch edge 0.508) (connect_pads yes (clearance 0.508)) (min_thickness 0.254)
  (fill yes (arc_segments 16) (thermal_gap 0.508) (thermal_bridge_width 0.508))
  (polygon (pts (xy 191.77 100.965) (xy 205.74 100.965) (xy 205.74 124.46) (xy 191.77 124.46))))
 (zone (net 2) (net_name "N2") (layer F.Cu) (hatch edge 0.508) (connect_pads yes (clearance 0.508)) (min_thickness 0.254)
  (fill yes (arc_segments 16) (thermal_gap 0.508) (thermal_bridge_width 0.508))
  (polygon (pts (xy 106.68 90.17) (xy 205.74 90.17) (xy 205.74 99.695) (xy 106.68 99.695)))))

